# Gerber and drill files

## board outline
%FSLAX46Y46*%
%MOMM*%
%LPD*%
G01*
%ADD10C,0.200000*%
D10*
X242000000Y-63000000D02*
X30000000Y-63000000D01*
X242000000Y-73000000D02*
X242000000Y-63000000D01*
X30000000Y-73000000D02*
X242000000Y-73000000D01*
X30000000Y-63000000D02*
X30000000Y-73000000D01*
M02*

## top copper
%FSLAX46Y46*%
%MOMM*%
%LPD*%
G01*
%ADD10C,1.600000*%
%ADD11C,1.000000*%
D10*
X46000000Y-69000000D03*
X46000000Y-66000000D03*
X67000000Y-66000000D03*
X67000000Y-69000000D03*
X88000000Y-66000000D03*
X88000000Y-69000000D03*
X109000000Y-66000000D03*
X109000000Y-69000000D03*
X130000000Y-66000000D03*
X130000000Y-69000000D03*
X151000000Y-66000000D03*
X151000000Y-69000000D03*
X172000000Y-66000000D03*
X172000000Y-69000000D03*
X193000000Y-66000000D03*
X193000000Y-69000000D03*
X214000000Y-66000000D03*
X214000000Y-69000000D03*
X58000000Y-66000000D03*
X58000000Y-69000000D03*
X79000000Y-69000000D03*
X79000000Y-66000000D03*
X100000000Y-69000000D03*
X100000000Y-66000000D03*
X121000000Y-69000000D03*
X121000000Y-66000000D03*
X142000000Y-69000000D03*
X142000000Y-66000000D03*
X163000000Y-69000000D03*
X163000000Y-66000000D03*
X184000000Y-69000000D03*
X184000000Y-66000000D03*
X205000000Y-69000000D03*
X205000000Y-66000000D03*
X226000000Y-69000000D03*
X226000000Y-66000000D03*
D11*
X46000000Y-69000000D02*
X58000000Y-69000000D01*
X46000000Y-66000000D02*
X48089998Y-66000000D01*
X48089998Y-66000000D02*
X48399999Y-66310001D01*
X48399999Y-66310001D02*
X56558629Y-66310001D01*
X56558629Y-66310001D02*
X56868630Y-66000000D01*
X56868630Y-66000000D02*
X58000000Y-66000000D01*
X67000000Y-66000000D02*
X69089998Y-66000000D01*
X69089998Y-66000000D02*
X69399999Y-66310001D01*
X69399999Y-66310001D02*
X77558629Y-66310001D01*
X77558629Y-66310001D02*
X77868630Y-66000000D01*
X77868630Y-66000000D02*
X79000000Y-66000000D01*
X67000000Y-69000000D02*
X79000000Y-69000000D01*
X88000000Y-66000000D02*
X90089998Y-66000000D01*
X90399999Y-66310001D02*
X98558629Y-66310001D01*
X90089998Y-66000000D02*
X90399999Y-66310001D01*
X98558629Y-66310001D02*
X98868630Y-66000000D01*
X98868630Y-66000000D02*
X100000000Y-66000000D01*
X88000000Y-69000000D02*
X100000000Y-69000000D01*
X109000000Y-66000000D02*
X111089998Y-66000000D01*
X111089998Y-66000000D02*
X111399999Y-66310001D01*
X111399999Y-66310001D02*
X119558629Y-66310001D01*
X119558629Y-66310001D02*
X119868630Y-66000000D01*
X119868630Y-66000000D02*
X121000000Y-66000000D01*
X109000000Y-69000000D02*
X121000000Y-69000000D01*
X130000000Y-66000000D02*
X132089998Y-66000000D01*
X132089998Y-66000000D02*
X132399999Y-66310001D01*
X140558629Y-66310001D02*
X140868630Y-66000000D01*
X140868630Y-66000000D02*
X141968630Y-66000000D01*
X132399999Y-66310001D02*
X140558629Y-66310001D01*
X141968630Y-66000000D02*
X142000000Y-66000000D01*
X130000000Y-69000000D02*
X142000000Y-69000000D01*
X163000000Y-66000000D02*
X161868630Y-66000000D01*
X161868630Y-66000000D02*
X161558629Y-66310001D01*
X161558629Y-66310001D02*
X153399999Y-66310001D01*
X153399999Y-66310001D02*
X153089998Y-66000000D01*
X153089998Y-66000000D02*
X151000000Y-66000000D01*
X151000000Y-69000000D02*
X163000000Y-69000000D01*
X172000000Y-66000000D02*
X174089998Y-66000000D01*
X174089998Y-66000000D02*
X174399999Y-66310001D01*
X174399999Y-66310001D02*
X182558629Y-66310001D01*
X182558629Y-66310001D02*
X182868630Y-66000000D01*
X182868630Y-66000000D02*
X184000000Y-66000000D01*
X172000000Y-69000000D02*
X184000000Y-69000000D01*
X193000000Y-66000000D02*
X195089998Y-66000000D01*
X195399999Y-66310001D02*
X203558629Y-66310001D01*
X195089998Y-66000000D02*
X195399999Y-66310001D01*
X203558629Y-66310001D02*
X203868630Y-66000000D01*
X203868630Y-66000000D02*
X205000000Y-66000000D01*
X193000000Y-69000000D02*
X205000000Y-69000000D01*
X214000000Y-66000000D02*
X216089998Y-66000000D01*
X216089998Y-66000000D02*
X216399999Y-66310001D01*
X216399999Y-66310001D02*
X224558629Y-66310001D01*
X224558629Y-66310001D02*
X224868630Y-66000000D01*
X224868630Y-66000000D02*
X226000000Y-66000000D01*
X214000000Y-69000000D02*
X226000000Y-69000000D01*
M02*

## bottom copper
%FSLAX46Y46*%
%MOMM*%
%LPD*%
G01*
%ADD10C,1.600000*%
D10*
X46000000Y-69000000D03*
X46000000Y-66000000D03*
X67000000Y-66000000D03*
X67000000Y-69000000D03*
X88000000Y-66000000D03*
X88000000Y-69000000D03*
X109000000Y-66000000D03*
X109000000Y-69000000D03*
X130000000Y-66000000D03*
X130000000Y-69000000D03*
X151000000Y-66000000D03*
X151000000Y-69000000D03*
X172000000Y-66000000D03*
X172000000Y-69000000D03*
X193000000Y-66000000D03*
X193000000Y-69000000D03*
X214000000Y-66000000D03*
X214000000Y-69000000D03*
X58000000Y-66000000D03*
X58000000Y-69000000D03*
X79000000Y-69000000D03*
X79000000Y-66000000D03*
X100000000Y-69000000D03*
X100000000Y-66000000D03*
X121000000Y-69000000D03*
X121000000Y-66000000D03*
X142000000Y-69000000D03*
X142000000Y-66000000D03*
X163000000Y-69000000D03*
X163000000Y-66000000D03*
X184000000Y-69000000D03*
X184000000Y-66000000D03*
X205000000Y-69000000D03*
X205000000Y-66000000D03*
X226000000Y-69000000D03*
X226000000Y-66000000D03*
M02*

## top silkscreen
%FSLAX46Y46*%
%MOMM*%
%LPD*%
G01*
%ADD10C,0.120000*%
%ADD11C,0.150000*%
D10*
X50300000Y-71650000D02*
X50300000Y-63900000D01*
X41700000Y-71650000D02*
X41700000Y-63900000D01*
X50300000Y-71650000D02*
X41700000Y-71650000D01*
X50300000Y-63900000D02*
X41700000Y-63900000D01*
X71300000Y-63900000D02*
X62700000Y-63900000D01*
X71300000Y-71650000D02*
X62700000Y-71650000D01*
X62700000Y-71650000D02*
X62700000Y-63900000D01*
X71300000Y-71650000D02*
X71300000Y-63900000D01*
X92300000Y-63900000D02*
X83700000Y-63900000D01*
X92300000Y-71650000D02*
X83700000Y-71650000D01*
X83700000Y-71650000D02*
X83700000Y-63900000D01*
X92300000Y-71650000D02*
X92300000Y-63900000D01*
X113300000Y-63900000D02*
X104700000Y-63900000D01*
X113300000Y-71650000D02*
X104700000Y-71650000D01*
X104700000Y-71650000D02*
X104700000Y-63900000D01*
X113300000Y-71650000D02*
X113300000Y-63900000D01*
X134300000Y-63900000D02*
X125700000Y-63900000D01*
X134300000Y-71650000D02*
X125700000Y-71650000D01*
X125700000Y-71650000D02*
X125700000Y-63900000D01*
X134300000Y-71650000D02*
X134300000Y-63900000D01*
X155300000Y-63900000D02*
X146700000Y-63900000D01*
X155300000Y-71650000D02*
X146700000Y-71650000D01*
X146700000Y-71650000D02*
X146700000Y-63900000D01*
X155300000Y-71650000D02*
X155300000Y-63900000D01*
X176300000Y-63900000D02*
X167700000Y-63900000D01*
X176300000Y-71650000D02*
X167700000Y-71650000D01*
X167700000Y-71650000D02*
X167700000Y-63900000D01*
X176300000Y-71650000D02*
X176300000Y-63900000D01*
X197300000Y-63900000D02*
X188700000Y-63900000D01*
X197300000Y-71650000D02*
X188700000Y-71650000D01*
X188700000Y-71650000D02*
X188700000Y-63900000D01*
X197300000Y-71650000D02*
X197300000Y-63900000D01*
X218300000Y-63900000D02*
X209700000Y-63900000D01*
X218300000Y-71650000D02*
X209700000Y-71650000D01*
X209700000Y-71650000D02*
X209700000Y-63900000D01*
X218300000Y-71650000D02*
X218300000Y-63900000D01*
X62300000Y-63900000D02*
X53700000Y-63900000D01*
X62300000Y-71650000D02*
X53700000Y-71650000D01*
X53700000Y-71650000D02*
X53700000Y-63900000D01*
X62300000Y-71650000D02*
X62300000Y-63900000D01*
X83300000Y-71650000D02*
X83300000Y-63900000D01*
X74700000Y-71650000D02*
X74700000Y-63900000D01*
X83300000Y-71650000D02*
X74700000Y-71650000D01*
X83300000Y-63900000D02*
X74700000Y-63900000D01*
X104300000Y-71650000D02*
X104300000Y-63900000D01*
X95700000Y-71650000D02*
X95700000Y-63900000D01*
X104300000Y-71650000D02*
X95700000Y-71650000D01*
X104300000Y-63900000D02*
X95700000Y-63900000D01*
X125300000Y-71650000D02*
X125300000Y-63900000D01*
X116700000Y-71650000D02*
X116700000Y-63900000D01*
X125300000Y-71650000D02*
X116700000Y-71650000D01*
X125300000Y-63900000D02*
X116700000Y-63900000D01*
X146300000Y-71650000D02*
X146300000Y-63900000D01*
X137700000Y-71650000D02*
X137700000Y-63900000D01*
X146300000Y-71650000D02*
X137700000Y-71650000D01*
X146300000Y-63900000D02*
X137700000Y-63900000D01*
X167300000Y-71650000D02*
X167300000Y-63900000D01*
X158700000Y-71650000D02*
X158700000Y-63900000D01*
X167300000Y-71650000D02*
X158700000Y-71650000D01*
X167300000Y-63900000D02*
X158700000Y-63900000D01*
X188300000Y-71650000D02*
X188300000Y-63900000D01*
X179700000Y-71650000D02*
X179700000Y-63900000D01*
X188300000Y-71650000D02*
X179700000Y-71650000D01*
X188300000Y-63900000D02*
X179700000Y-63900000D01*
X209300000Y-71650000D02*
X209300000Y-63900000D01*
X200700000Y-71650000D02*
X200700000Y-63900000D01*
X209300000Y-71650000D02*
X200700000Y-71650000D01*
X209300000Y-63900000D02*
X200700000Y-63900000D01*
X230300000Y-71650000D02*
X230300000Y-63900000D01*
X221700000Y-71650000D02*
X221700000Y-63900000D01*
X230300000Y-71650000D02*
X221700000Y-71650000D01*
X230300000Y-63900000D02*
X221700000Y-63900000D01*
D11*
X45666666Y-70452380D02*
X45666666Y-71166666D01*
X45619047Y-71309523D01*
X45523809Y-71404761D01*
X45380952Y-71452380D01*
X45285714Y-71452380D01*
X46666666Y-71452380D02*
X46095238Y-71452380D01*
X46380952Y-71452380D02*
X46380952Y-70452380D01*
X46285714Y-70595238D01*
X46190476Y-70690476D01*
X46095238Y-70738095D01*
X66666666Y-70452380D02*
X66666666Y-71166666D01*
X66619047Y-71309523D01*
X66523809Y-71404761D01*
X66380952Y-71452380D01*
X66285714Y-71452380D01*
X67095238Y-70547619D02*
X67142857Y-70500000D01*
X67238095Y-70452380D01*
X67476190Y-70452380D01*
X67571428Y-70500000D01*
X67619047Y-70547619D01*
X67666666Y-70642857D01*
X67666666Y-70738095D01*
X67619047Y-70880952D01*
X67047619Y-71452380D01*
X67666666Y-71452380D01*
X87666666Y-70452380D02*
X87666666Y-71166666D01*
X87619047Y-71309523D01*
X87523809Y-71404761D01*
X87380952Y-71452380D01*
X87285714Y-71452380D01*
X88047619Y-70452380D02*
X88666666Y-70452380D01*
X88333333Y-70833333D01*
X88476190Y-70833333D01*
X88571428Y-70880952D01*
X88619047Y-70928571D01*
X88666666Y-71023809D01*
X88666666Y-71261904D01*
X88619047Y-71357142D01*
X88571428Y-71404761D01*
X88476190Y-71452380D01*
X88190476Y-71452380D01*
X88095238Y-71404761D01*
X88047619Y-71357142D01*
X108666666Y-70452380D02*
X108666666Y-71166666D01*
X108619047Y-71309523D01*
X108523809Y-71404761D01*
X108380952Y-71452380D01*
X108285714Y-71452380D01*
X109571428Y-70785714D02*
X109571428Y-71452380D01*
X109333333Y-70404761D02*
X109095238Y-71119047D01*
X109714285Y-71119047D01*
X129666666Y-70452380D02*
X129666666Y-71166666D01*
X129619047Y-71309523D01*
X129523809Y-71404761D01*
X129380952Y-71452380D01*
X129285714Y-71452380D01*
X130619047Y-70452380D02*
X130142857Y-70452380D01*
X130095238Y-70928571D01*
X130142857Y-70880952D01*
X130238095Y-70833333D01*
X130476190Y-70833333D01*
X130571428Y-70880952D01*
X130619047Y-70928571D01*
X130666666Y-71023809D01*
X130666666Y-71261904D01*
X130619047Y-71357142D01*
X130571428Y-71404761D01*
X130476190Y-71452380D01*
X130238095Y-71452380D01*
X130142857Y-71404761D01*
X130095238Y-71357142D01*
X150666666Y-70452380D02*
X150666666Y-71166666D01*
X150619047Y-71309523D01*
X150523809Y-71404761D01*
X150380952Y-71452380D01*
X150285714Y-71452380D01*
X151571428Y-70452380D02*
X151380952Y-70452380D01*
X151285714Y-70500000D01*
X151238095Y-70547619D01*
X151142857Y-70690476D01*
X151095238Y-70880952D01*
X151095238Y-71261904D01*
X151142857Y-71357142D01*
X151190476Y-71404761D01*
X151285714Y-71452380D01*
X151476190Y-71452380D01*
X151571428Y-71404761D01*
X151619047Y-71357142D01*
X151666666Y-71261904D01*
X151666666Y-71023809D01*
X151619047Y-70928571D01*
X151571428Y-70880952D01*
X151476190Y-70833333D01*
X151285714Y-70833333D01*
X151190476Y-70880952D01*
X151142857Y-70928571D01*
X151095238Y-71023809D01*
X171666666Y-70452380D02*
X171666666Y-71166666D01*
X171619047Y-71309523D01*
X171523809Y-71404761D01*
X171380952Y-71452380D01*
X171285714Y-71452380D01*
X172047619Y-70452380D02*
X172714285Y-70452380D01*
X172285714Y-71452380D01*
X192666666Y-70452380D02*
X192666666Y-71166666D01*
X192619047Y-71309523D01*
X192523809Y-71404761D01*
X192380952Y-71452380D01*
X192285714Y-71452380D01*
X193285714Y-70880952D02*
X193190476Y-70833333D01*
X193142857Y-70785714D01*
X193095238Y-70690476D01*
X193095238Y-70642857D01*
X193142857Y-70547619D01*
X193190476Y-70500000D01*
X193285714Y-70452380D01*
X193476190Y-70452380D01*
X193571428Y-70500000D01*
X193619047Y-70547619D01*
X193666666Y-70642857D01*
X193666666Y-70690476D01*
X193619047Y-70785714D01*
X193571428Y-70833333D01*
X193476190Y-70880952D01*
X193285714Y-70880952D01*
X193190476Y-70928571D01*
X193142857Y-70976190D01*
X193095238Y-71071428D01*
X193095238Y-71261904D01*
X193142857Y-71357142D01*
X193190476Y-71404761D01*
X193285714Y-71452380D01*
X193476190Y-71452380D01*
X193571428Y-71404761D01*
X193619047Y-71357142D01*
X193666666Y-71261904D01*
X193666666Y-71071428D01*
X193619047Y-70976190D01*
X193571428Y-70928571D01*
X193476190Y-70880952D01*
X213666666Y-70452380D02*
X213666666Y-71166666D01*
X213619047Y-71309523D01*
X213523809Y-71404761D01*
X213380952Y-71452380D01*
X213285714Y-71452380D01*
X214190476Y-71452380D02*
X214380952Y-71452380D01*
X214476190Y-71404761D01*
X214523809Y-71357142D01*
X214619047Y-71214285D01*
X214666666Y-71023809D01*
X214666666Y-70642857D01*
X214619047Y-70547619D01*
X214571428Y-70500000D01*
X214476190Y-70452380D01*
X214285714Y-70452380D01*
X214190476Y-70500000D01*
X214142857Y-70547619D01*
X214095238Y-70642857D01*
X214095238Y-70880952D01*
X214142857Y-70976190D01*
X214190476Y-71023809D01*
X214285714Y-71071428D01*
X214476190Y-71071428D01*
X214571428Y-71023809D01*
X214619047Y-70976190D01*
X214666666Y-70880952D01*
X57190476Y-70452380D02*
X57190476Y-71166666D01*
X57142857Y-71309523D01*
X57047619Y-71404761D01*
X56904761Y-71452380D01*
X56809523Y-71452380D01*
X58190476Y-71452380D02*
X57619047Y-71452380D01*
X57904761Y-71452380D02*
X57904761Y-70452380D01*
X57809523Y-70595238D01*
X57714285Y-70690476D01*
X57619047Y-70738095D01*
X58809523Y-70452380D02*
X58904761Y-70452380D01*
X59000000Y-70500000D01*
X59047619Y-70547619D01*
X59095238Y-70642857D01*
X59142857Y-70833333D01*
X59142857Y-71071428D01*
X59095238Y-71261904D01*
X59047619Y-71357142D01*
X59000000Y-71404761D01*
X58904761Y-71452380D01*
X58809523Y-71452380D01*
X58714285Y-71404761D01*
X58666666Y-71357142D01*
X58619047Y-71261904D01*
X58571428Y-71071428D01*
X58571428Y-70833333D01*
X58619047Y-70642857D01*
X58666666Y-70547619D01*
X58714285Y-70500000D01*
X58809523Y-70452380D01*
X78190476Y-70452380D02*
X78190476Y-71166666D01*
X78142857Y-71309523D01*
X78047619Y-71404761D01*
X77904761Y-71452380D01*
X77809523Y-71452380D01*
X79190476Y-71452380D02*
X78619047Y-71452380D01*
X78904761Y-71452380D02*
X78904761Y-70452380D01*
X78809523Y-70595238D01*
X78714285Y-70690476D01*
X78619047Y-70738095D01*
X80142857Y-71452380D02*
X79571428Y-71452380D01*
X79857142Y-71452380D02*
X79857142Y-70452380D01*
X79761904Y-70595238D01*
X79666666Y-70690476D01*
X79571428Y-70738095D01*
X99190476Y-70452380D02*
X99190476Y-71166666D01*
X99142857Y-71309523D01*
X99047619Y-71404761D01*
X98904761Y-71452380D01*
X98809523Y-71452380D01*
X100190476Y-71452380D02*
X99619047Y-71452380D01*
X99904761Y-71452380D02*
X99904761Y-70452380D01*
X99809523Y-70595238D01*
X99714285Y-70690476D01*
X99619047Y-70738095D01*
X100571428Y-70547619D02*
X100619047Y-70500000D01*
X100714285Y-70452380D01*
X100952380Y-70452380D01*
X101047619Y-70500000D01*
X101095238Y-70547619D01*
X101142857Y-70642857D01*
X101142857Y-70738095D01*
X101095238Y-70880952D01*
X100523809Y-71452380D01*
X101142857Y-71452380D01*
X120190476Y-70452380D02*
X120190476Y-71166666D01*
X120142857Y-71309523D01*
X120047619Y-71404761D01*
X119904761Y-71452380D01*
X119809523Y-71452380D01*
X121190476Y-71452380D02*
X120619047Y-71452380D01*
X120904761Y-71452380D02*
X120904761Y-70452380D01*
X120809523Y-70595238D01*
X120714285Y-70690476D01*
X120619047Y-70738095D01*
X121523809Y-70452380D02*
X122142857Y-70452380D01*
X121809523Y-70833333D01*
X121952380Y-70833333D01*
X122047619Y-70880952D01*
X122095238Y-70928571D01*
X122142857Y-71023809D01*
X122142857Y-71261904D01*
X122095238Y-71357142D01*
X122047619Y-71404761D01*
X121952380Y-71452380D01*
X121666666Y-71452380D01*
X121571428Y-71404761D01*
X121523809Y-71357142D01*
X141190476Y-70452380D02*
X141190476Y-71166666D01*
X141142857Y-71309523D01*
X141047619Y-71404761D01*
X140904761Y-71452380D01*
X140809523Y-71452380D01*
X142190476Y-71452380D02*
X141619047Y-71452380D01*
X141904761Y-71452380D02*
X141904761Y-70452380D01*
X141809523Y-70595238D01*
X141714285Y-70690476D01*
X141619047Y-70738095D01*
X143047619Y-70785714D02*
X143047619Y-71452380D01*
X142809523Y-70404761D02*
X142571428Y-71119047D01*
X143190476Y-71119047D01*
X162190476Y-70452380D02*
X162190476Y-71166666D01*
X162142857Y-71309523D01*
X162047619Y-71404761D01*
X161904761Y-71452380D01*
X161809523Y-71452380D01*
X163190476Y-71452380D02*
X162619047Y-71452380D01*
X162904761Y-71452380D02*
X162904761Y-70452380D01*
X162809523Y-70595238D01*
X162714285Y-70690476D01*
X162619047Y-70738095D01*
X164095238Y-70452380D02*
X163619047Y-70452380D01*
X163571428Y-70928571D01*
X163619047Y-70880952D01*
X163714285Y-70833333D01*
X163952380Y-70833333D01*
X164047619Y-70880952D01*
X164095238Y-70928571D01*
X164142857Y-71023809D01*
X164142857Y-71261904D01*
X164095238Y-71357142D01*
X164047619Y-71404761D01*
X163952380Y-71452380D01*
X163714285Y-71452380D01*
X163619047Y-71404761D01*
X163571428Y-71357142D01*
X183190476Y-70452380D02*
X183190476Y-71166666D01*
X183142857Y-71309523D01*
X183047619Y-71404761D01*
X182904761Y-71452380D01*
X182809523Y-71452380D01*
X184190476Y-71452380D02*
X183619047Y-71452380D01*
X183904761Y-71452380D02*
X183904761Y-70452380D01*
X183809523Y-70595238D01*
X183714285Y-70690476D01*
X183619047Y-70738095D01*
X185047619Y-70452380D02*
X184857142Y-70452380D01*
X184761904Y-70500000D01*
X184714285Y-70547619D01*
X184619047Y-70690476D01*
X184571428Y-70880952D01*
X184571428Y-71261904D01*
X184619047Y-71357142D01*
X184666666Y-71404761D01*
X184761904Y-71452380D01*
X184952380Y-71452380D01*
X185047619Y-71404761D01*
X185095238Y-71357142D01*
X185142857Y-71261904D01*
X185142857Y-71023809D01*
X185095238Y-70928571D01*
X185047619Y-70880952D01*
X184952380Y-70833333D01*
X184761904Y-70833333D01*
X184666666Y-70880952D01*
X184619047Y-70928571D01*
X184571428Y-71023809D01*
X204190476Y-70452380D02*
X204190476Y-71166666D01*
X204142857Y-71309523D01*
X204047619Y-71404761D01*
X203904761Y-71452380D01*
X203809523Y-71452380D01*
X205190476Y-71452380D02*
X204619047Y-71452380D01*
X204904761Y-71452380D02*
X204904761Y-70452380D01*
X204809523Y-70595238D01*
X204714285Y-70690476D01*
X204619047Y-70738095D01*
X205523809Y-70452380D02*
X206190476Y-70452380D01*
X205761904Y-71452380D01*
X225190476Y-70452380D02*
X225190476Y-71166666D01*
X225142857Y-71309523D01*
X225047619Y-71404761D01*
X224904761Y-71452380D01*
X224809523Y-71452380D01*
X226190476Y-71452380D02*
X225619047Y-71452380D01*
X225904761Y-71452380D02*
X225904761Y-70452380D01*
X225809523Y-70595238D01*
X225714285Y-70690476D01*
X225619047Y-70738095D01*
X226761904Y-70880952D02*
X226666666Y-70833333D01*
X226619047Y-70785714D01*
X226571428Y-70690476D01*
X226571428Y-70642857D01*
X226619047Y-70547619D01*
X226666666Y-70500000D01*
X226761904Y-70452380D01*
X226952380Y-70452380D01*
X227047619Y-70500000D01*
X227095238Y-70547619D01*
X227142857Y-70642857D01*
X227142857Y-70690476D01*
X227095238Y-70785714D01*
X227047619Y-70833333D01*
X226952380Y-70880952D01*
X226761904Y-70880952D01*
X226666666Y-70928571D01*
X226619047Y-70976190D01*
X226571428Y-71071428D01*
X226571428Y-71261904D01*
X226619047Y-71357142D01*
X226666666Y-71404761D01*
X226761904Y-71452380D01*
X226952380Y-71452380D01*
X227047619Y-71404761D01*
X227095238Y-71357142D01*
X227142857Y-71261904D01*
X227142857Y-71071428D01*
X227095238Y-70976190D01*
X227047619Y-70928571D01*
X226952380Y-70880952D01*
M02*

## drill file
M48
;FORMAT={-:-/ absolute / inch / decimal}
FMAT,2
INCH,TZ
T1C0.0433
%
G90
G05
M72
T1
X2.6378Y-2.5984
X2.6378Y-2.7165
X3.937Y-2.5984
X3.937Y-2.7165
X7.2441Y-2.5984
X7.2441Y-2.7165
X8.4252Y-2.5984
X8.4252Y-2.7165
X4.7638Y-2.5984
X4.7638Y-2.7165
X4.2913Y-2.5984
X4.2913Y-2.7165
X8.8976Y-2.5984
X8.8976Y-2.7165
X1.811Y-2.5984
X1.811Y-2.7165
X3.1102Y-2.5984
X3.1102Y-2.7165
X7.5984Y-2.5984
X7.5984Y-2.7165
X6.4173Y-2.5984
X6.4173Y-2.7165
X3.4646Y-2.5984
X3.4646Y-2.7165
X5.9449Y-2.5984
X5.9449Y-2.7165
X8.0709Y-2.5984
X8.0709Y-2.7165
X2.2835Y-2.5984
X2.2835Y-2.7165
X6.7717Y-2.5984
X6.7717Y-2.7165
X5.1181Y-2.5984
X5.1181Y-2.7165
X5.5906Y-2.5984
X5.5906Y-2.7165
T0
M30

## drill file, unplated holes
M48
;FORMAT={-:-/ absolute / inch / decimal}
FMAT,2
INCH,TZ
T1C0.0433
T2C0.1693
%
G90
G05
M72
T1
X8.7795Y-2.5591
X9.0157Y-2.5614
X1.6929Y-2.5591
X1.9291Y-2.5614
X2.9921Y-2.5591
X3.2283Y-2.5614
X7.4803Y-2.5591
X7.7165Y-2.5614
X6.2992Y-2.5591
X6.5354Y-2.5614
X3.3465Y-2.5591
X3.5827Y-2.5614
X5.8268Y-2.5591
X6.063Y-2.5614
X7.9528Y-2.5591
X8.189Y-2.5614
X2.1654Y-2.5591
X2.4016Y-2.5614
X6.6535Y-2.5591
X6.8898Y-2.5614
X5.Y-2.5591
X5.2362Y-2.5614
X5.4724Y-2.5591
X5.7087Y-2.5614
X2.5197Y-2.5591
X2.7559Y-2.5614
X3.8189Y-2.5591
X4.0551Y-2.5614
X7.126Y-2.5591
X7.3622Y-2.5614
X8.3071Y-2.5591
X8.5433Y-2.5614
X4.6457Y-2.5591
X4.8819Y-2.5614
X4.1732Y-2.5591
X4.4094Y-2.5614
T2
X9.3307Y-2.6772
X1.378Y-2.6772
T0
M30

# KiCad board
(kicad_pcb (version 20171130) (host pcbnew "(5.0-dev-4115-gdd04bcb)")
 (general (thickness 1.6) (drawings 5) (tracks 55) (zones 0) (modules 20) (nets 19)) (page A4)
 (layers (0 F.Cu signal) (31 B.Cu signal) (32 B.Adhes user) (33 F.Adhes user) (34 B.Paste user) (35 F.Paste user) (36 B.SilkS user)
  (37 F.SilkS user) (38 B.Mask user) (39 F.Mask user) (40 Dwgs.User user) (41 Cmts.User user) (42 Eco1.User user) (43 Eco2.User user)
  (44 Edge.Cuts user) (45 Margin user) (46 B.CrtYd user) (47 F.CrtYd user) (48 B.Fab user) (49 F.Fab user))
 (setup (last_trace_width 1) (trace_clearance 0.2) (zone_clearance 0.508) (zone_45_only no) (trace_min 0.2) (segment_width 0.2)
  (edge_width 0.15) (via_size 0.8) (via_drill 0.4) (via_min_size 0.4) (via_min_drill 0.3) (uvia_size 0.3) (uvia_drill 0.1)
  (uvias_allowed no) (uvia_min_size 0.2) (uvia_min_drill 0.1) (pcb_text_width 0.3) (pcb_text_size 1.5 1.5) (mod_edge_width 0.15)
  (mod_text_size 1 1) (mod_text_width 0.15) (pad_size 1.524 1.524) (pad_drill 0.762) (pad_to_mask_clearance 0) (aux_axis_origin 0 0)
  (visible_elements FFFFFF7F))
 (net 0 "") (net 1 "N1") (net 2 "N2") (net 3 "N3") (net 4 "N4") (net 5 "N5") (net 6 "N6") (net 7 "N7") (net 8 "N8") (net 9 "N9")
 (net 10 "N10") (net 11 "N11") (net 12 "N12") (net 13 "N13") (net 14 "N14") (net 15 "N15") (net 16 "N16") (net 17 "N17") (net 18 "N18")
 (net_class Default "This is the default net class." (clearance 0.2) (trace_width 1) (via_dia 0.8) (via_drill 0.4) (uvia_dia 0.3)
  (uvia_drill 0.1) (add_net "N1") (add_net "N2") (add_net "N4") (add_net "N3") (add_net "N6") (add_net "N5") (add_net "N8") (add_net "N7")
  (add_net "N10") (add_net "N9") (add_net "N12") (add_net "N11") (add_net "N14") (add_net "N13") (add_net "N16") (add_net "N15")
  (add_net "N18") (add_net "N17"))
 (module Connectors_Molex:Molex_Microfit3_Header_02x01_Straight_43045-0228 (layer F.Cu) (at 46 69)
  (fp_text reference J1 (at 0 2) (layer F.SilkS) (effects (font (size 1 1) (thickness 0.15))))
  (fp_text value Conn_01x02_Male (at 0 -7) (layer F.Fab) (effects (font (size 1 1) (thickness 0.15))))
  (fp_line (start 4.3 2.65) (end 4.3 -5.1) (layer F.SilkS) (width 0.12))
  (fp_line (start -4.3 2.65) (end -4.3 -5.1) (layer F.SilkS) (width 0.12))
  (fp_line (start 4.3 2.65) (end -4.3 2.65) (layer F.SilkS) (width 0.12))
  (fp_line (start 4.3 -5.1) (end -4.3 -5.1) (layer F.SilkS) (width 0.12))
  (pad "" np_thru_hole circle (at -3 -4) (size 1.1 1.1) (drill 1.1) (layers *.Cu *.Mask))
  (pad 1 thru_hole circle (at 0 0) (size 1.6 1.6) (drill 1.1) (layers *.Cu *.Mask) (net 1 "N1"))
  (pad 2 thru_hole circle (at 0 -3) (size 1.6 1.6) (drill 1.1) (layers *.Cu *.Mask) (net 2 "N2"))
  (pad "" np_thru_hole circle (at 3 -3.94) (size 1.1 1.1) (drill 1.1) (layers *.Cu *.Mask)))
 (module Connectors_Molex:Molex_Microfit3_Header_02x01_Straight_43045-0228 (layer F.Cu) (at 67 69)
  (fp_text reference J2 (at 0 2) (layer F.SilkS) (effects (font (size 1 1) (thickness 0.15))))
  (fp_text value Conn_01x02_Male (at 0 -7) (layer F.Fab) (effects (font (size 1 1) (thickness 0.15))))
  (fp_line (start 4.3 -5.1) (end -4.3 -5.1) (layer F.SilkS) (width 0.12))
  (fp_line (start 4.3 2.65) (end -4.3 2.65) (layer F.SilkS) (width 0.12))
  (fp_line (start -4.3 2.65) (end -4.3 -5.1) (layer F.SilkS) (width 0.12))
  (fp_line (start 4.3 2.65) (end 4.3 -5.1) (layer F.SilkS) (width 0.12))
  (pad "" np_thru_hole circle (at 3 -3.94) (size 1.1 1.1) (drill 1.1) (layers *.Cu *.Mask))
  (pad 2 thru_hole circle (at 0 -3) (size 1.6 1.6) (drill 1.1) (layers *.Cu *.Mask) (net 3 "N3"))
  (pad 1 thru_hole circle (at 0 0) (size 1.6 1.6) (drill 1.1) (layers *.Cu *.Mask) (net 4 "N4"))
  (pad "" np_thru_hole circle (at -3 -4) (size 1.1 1.1) (drill 1.1) (layers *.Cu *.Mask)))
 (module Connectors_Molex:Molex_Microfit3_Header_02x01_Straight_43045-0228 (layer F.Cu) (at 88 69)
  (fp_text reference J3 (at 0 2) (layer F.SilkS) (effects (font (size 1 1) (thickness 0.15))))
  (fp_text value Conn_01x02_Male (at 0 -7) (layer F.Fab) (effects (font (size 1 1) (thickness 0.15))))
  (fp_line (start 4.3 -5.1) (end -4.3 -5.1) (layer F.SilkS) (width 0.12))
  (fp_line (start 4.3 2.65) (end -4.3 2.65) (layer F.SilkS) (width 0.12))
  (fp_line (start -4.3 2.65) (end -4.3 -5.1) (layer F.SilkS) (width 0.12))
  (fp_line (start 4.3 2.65) (end 4.3 -5.1) (layer F.SilkS) (width 0.12))
  (pad "" np_thru_hole circle (at 3 -3.94) (size 1.1 1.1) (drill 1.1) (layers *.Cu *.Mask))
  (pad 2 thru_hole circle (at 0 -3) (size 1.6 1.6) (drill 1.1) (layers *.Cu *.Mask) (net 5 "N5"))
  (pad 1 thru_hole circle (at 0 0) (size 1.6 1.6) (drill 1.1) (layers *.Cu *.Mask) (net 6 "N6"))
  (pad "" np_thru_hole circle (at -3 -4) (size 1.1 1.1) (drill 1.1) (layers *.Cu *.Mask)))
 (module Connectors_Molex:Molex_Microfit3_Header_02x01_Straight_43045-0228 (layer F.Cu) (at 109 69)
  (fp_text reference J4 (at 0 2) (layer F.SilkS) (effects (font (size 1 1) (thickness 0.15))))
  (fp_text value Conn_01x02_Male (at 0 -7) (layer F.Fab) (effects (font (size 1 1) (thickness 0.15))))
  (fp_line (start 4.3 -5.1) (end -4.3 -5.1) (layer F.SilkS) (width 0.12))
  (fp_line (start 4.3 2.65) (end -4.3 2.65) (layer F.SilkS) (width 0.12))
  (fp_line (start -4.3 2.65) (end -4.3 -5.1) (layer F.SilkS) (width 0.12))
  (fp_line (start 4.3 2.65) (end 4.3 -5.1) (layer F.SilkS) (width 0.12))
  (pad "" np_thru_hole circle (at 3 -3.94) (size 1.1 1.1) (drill 1.1) (layers *.Cu *.Mask))
  (pad 2 thru_hole circle (at 0 -3) (size 1.6 1.6) (drill 1.1) (layers *.Cu *.Mask) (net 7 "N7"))
  (pad 1 thru_hole circle (at 0 0) (size 1.6 1.6) (drill 1.1) (layers *.Cu *.Mask) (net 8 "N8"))
  (pad "" np_thru_hole circle (at -3 -4) (size 1.1 1.1) (drill 1.1) (layers *.Cu *.Mask)))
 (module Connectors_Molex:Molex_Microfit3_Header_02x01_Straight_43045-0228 (layer F.Cu) (at 130 69)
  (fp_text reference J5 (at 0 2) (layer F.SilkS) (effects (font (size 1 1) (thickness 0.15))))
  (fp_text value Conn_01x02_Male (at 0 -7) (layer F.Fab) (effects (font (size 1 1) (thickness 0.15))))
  (fp_line (start 4.3 -5.1) (end -4.3 -5.1) (layer F.SilkS) (width 0.12))
  (fp_line (start 4.3 2.65) (end -4.3 2.65) (layer F.SilkS) (width 0.12))
  (fp_line (start -4.3 2.65) (end -4.3 -5.1) (layer F.SilkS) (width 0.12))
  (fp_line (start 4.3 2.65) (end 4.3 -5.1) (layer F.SilkS) (width 0.12))
  (pad "" np_thru_hole circle (at 3 -3.94) (size 1.1 1.1) (drill 1.1) (layers *.Cu *.Mask))
  (pad 2 thru_hole circle (at 0 -3) (size 1.6 1.6) (drill 1.1) (layers *.Cu *.Mask) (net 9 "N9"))
  (pad 1 thru_hole circle (at 0 0) (size 1.6 1.6) (drill 1.1) (layers *.Cu *.Mask) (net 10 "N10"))
  (pad "" np_thru_hole circle (at -3 -4) (size 1.1 1.1) (drill 1.1) (layers *.Cu *.Mask)))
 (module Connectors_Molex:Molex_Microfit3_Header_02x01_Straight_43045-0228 (layer F.Cu) (at 151 69)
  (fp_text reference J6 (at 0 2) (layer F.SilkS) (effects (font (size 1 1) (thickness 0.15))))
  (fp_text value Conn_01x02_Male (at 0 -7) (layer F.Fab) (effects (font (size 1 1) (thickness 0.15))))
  (fp_line (start 4.3 -5.1) (end -4.3 -5.1) (layer F.SilkS) (width 0.12))
  (fp_line (start 4.3 2.65) (end -4.3 2.65) (layer F.SilkS) (width 0.12))
  (fp_line (start -4.3 2.65) (end -4.3 -5.1) (layer F.SilkS) (width 0.12))
  (fp_line (start 4.3 2.65) (end 4.3 -5.1) (layer F.SilkS) (width 0.12))
  (pad "" np_thru_hole circle (at 3 -3.94) (size 1.1 1.1) (drill 1.1) (layers *.Cu *.Mask))
  (pad 2 thru_hole circle (at 0 -3) (size 1.6 1.6) (drill 1.1) (layers *.Cu *.Mask) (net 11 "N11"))
  (pad 1 thru_hole circle (at 0 0) (size 1.6 1.6) (drill 1.1) (layers *.Cu *.Mask) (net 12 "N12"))
  (pad "" np_thru_hole circle (at -3 -4) (size 1.1 1.1) (drill 1.1) (layers *.Cu *.Mask)))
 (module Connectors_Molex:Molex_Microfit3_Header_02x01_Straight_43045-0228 (layer F.Cu) (at 172 69)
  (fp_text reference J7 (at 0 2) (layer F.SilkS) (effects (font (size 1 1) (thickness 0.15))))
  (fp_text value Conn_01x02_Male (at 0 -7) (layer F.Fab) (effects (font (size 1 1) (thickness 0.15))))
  (fp_line (start 4.3 -5.1) (end -4.3 -5.1) (layer F.SilkS) (width 0.12))
  (fp_line (start 4.3 2.65) (end -4.3 2.65) (layer F.SilkS) (width 0.12))
  (fp_line (start -4.3 2.65) (end -4.3 -5.1) (layer F.SilkS) (width 0.12))
  (fp_line (start 4.3 2.65) (end 4.3 -5.1) (layer F.SilkS) (width 0.12))
  (pad "" np_thru_hole circle (at 3 -3.94) (size 1.1 1.1) (drill 1.1) (layers *.Cu *.Mask))
  (pad 2 thru_hole circle (at 0 -3) (size 1.6 1.6) (drill 1.1) (layers *.Cu *.Mask) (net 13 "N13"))
  (pad 1 thru_hole circle (at 0 0) (size 1.6 1.6) (drill 1.1) (layers *.Cu *.Mask) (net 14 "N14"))
  (pad "" np_thru_hole circle (at -3 -4) (size 1.1 1.1) (drill 1.1) (layers *.Cu *.Mask)))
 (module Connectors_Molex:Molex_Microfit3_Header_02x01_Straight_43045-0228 (layer F.Cu) (at 193 69)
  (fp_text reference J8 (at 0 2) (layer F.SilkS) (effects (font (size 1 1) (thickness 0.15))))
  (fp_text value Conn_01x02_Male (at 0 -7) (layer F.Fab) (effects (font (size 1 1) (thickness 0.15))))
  (fp_line (start 4.3 -5.1) (end -4.3 -5.1) (layer F.SilkS) (width 0.12))
  (fp_line (start 4.3 2.65) (end -4.3 2.65) (layer F.SilkS) (width 0.12))
  (fp_line (start -4.3 2.65) (end -4.3 -5.1) (layer F.SilkS) (width 0.12))
  (fp_line (start 4.3 2.65) (end 4.3 -5.1) (layer F.SilkS) (width 0.12))
  (pad "" np_thru_hole circle (at 3 -3.94) (size 1.1 1.1) (drill 1.1) (layers *.Cu *.Mask))
  (pad 2 thru_hole circle (at 0 -3) (size 1.6 1.6) (drill 1.1) (layers *.Cu *.Mask) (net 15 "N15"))
  (pad 1 thru_hole circle (at 0 0) (size 1.6 1.6) (drill 1.1) (layers *.Cu *.Mask) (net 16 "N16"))
  (pad "" np_thru_hole circle (at -3 -4) (size 1.1 1.1) (drill 1.1) (layers *.Cu *.Mask)))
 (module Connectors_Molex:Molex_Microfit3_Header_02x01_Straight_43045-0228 (layer F.Cu) (at 214 69)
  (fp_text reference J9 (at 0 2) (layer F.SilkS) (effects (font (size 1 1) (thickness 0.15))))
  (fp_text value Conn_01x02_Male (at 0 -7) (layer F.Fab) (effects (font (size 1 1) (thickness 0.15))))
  (fp_line (start 4.3 -5.1) (end -4.3 -5.1) (layer F.SilkS) (width 0.12))
  (fp_line (start 4.3 2.65) (end -4.3 2.65) (layer F.SilkS) (width 0.12))
  (fp_line (start -4.3 2.65) (end -4.3 -5.1) (layer F.SilkS) (width 0.12))
  (fp_line (start 4.3 2.65) (end 4.3 -5.1) (layer F.SilkS) (width 0.12))
  (pad "" np_thru_hole circle (at 3 -3.94) (size 1.1 1.1) (drill 1.1) (layers *.Cu *.Mask))
  (pad 2 thru_hole circle (at 0 -3) (size 1.6 1.6) (drill 1.1) (layers *.Cu *.Mask) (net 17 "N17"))
  (pad 1 thru_hole circle (at 0 0) (size 1.6 1.6) (drill 1.1) (layers *.Cu *.Mask) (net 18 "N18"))
  (pad "" np_thru_hole circle (at -3 -4) (size 1.1 1.1) (drill 1.1) (layers *.Cu *.Mask)))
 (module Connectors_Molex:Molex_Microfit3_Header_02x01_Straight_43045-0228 (layer F.Cu) (at 58 69)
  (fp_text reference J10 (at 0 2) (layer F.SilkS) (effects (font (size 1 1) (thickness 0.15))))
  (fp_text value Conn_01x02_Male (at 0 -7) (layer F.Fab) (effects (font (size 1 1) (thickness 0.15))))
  (fp_line (start 4.3 -5.1) (end -4.3 -5.1) (layer F.SilkS) (width 0.12))
  (fp_line (start 4.3 2.65) (end -4.3 2.65) (layer F.SilkS) (width 0.12))
  (fp_line (start -4.3 2.65) (end -4.3 -5.1) (layer F.SilkS) (width 0.12))
  (fp_line (start 4.3 2.65) (end 4.3 -5.1) (layer F.SilkS) (width 0.12))
  (pad "" np_thru_hole circle (at 3 -3.94) (size 1.1 1.1) (drill 1.1) (layers *.Cu *.Mask))
  (pad 2 thru_hole circle (at 0 -3) (size 1.6 1.6) (drill 1.1) (layers *.Cu *.Mask) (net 2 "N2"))
  (pad 1 thru_hole circle (at 0 0) (size 1.6 1.6) (drill 1.1) (layers *.Cu *.Mask) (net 1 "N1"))
  (pad "" np_thru_hole circle (at -3 -4) (size 1.1 1.1) (drill 1.1) (layers *.Cu *.Mask)))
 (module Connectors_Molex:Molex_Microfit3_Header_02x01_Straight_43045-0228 (layer F.Cu) (at 79 69)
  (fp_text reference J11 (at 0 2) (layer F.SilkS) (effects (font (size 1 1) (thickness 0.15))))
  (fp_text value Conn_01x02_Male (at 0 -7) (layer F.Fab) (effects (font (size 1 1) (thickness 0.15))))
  (fp_line (start 4.3 2.65) (end 4.3 -5.1) (layer F.SilkS) (width 0.12))
  (fp_line (start -4.3 2.65) (end -4.3 -5.1) (layer F.SilkS) (width 0.12))
  (fp_line (start 4.3 2.65) (end -4.3 2.65) (layer F.SilkS) (width 0.12))
  (fp_line (start 4.3 -5.1) (end -4.3 -5.1) (layer F.SilkS) (width 0.12))
  (pad "" np_thru_hole circle (at -3 -4) (size 1.1 1.1) (drill 1.1) (layers *.Cu *.Mask))
  (pad 1 thru_hole circle (at 0 0) (size 1.6 1.6) (drill 1.1) (layers *.Cu *.Mask) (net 4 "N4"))
  (pad 2 thru_hole circle (at 0 -3) (size 1.6 1.6) (drill 1.1) (layers *.Cu *.Mask) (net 3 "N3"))
  (pad "" np_thru_hole circle (at 3 -3.94) (size 1.1 1.1) (drill 1.1) (layers *.Cu *.Mask)))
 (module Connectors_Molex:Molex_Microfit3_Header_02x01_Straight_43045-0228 (layer F.Cu) (at 100 69)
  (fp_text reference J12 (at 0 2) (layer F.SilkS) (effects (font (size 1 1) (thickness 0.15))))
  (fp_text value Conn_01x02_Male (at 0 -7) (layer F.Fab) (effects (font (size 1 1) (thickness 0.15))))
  (fp_line (start 4.3 2.65) (end 4.3 -5.1) (layer F.SilkS) (width 0.12))
  (fp_line (start -4.3 2.65) (end -4.3 -5.1) (layer F.SilkS) (width 0.12))
  (fp_line (start 4.3 2.65) (end -4.3 2.65) (layer F.SilkS) (width 0.12))
  (fp_line (start 4.3 -5.1) (end -4.3 -5.1) (layer F.SilkS) (width 0.12))
  (pad "" np_thru_hole circle (at -3 -4) (size 1.1 1.1) (drill 1.1) (layers *.Cu *.Mask))
  (pad 1 thru_hole circle (at 0 0) (size 1.6 1.6) (drill 1.1) (layers *.Cu *.Mask) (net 6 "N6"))
  (pad 2 thru_hole circle (at 0 -3) (size 1.6 1.6) (drill 1.1) (layers *.Cu *.Mask) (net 5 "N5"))
  (pad "" np_thru_hole circle (at 3 -3.94) (size 1.1 1.1) (drill 1.1) (layers *.Cu *.Mask)))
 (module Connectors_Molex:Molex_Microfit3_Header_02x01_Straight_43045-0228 (layer F.Cu) (at 121 69)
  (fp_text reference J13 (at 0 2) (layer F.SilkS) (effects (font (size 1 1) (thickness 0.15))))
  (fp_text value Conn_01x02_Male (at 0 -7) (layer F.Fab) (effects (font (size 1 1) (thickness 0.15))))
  (fp_line (start 4.3 2.65) (end 4.3 -5.1) (layer F.SilkS) (width 0.12))
  (fp_line (start -4.3 2.65) (end -4.3 -5.1) (layer F.SilkS) (width 0.12))
  (fp_line (start 4.3 2.65) (end -4.3 2.65) (layer F.SilkS) (width 0.12))
  (fp_line (start 4.3 -5.1) (end -4.3 -5.1) (layer F.SilkS) (width 0.12))
  (pad "" np_thru_hole circle (at -3 -4) (size 1.1 1.1) (drill 1.1) (layers *.Cu *.Mask))
  (pad 1 thru_hole circle (at 0 0) (size 1.6 1.6) (drill 1.1) (layers *.Cu *.Mask) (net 8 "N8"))
  (pad 2 thru_hole circle (at 0 -3) (size 1.6 1.6) (drill 1.1) (layers *.Cu *.Mask) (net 7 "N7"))
  (pad "" np_thru_hole circle (at 3 -3.94) (size 1.1 1.1) (drill 1.1) (layers *.Cu *.Mask)))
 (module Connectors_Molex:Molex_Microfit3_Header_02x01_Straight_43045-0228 (layer F.Cu) (at 142 69)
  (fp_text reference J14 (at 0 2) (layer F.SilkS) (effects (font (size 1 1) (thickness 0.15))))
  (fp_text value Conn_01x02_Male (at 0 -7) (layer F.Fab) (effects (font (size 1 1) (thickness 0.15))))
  (fp_line (start 4.3 2.65) (end 4.3 -5.1) (layer F.SilkS) (width 0.12))
  (fp_line (start -4.3 2.65) (end -4.3 -5.1) (layer F.SilkS) (width 0.12))
  (fp_line (start 4.3 2.65) (end -4.3 2.65) (layer F.SilkS) (width 0.12))
  (fp_line (start 4.3 -5.1) (end -4.3 -5.1) (layer F.SilkS) (width 0.12))
  (pad "" np_thru_hole circle (at -3 -4) (size 1.1 1.1) (drill 1.1) (layers *.Cu *.Mask))
  (pad 1 thru_hole circle (at 0 0) (size 1.6 1.6) (drill 1.1) (layers *.Cu *.Mask) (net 10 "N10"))
  (pad 2 thru_hole circle (at 0 -3) (size 1.6 1.6) (drill 1.1) (layers *.Cu *.Mask) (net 9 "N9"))
  (pad "" np_thru_hole circle (at 3 -3.94) (size 1.1 1.1) (drill 1.1) (layers *.Cu *.Mask)))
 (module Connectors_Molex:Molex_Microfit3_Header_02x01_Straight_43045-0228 (layer F.Cu) (at 163 69)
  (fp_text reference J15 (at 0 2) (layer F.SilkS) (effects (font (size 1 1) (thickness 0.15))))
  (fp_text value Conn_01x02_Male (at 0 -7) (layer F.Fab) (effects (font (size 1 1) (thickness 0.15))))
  (fp_line (start 4.3 2.65) (end 4.3 -5.1) (layer F.SilkS) (width 0.12))
  (fp_line (start -4.3 2.65) (end -4.3 -5.1) (layer F.SilkS) (width 0.12))
  (fp_line (start 4.3 2.65) (end -4.3 2.65) (layer F.SilkS) (width 0.12))
  (fp_line (start 4.3 -5.1) (end -4.3 -5.1) (layer F.SilkS) (width 0.12))
  (pad "" np_thru_hole circle (at -3 -4) (size 1.1 1.1) (drill 1.1) (layers *.Cu *.Mask))
  (pad 1 thru_hole circle (at 0 0) (size 1.6 1.6) (drill 1.1) (layers *.Cu *.Mask) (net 12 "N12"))
  (pad 2 thru_hole circle (at 0 -3) (size 1.6 1.6) (drill 1.1) (layers *.Cu *.Mask) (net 11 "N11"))
  (pad "" np_thru_hole circle (at 3 -3.94) (size 1.1 1.1) (drill 1.1) (layers *.Cu *.Mask)))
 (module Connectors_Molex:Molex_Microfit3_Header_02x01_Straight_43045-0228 (layer F.Cu) (at 184 69)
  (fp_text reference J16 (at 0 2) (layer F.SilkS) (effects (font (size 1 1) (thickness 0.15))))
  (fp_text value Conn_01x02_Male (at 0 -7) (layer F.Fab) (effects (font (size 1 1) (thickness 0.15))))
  (fp_line (start 4.3 2.65) (end 4.3 -5.1) (layer F.SilkS) (width 0.12))
  (fp_line (start -4.3 2.65) (end -4.3 -5.1) (layer F.SilkS) (width 0.12))
  (fp_line (start 4.3 2.65) (end -4.3 2.65) (layer F.SilkS) (width 0.12))
  (fp_line (start 4.3 -5.1) (end -4.3 -5.1) (layer F.SilkS) (width 0.12))
  (pad "" np_thru_hole circle (at -3 -4) (size 1.1 1.1) (drill 1.1) (layers *.Cu *.Mask))
  (pad 1 thru_hole circle (at 0 0) (size 1.6 1.6) (drill 1.1) (layers *.Cu *.Mask) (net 14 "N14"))
  (pad 2 thru_hole circle (at 0 -3) (size 1.6 1.6) (drill 1.1) (layers *.Cu *.Mask) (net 13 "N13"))
  (pad "" np_thru_hole circle (at 3 -3.94) (size 1.1 1.1) (drill 1.1) (layers *.Cu *.Mask)))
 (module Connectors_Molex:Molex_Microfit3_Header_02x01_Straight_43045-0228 (layer F.Cu) (at 205 69)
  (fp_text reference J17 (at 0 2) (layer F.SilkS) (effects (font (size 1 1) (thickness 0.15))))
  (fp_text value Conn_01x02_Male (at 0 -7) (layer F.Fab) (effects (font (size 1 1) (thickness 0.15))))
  (fp_line (start 4.3 2.65) (end 4.3 -5.1) (layer F.SilkS) (width 0.12))
  (fp_line (start -4.3 2.65) (end -4.3 -5.1) (layer F.SilkS) (width 0.12))
  (fp_line (start 4.3 2.65) (end -4.3 2.65) (layer F.SilkS) (width 0.12))
  (fp_line (start 4.3 -5.1) (end -4.3 -5.1) (layer F.SilkS) (width 0.12))
  (pad "" np_thru_hole circle (at -3 -4) (size 1.1 1.1) (drill 1.1) (layers *.Cu *.Mask))
  (pad 1 thru_hole circle (at 0 0) (size 1.6 1.6) (drill 1.1) (layers *.Cu *.Mask) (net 16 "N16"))
  (pad 2 thru_hole circle (at 0 -3) (size 1.6 1.6) (drill 1.1) (layers *.Cu *.Mask) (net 15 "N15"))
  (pad "" np_thru_hole circle (at 3 -3.94) (size 1.1 1.1) (drill 1.1) (layers *.Cu *.Mask)))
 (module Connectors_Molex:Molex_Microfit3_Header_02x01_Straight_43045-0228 (layer F.Cu) (at 226 69)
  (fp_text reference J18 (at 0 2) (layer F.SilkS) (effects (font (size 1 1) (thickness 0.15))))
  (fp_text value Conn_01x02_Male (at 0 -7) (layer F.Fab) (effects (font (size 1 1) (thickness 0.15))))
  (fp_line (start 4.3 2.65) (end 4.3 -5.1) (layer F.SilkS) (width 0.12))
  (fp_line (start -4.3 2.65) (end -4.3 -5.1) (layer F.SilkS) (width 0.12))
  (fp_line (start 4.3 2.65) (end -4.3 2.65) (layer F.SilkS) (width 0.12))
  (fp_line (start 4.3 -5.1) (end -4.3 -5.1) (layer F.SilkS) (width 0.12))
  (pad "" np_thru_hole circle (at -3 -4) (size 1.1 1.1) (drill 1.1) (layers *.Cu *.Mask))
  (pad 1 thru_hole circle (at 0 0) (size 1.6 1.6) (drill 1.1) (layers *.Cu *.Mask) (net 18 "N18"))
  (pad 2 thru_hole circle (at 0 -3) (size 1.6 1.6) (drill 1.1) (layers *.Cu *.Mask) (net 17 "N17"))
  (pad "" np_thru_hole circle (at 3 -3.94) (size 1.1 1.1) (drill 1.1) (layers *.Cu *.Mask)))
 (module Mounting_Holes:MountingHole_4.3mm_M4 (layer F.Cu) (at 35 68)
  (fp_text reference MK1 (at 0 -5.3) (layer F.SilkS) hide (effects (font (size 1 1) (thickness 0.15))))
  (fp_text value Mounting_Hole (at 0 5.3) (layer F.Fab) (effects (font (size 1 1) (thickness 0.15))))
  (pad 1 np_thru_hole circle (at 0 0) (size 4.3 4.3) (drill 4.3) (layers *.Cu *.Mask)))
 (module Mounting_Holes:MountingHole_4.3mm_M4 (layer F.Cu) (at 237 68)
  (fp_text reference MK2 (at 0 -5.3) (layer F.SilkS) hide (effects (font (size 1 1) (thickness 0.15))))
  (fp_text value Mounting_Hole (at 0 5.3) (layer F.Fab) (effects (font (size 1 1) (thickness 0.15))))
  (pad 1 np_thru_hole circle (at 0 0) (size 4.3 4.3) (drill 4.3) (layers *.Cu *.Mask)))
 (gr_line (start 242 63) (end 30 63) (layer Edge.Cuts) (width 0.2))
 (gr_line (start 242 73) (end 242 63) (layer Edge.Cuts) (width 0.2))
 (gr_line (start 30 73) (end 242 73) (layer Edge.Cuts) (width 0.2))
 (gr_line (start 30 63) (end 30 73) (layer Edge.Cuts) (width 0.2))
 (segment (start 46 69) (end 58 69) (width 1) (layer F.Cu) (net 1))
 (segment (start 46 66) (end 48.089998 66) (width 1) (layer F.Cu) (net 2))
 (segment (start 48.089998 66) (end 48.399999 66.310001) (width 1) (layer F.Cu) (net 2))
 (segment (start 48.399999 66.310001) (end 56.558629 66.310001) (width 1) (layer F.Cu) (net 2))
 (segment (start 56.558629 66.310001) (end 56.86863 66) (width 1) (layer F.Cu) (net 2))
 (segment (start 56.86863 66) (end 58 66) (width 1) (layer F.Cu) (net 2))
 (segment (start 67 66) (end 69.089998 66) (width 1) (layer F.Cu) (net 3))
 (segment (start 69.089998 66) (end 69.399999 66.310001) (width 1) (layer F.Cu) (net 3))
 (segment (start 69.399999 66.310001) (end 77.558629 66.310001) (width 1) (layer F.Cu) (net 3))
 (segment (start 77.558629 66.310001) (end 77.86863 66) (width 1) (layer F.Cu) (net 3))
 (segment (start 77.86863 66) (end 79 66) (width 1) (layer F.Cu) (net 3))
 (segment (start 67 69) (end 79 69) (width 1) (layer F.Cu) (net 4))
 (segment (start 88 66) (end 90.089998 66) (width 1) (layer F.Cu) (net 5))
 (segment (start 90.399999 66.310001) (end 98.558629 66.310001) (width 1) (layer F.Cu) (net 5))
 (segment (start 90.089998 66) (end 90.399999 66.310001) (width 1) (layer F.Cu) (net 5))
 (segment (start 98.558629 66.310001) (end 98.86863 66) (width 1) (layer F.Cu) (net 5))
 (segment (start 98.86863 66) (end 100 66) (width 1) (layer F.Cu) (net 5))
 (segment (start 88 69) (end 100 69) (width 1) (layer F.Cu) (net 6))
 (segment (start 109 66) (end 111.089998 66) (width 1) (layer F.Cu) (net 7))
 (segment (start 111.089998 66) (end 111.399999 66.310001) (width 1) (layer F.Cu) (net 7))
 (segment (start 111.399999 66.310001) (end 119.558629 66.310001) (width 1) (layer F.Cu) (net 7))
 (segment (start 119.558629 66.310001) (end 119.86863 66) (width 1) (layer F.Cu) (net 7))
 (segment (start 119.86863 66) (end 121 66) (width 1) (layer F.Cu) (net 7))
 (segment (start 109 69) (end 121 69) (width 1) (layer F.Cu) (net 8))
 (segment (start 130 66) (end 132.089998 66) (width 1) (layer F.Cu) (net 9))
 (segment (start 132.089998 66) (end 132.399999 66.310001) (width 1) (layer F.Cu) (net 9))
 (segment (start 140.558629 66.310001) (end 140.86863 66) (width 1) (layer F.Cu) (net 9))
 (segment (start 140.86863 66) (end 141.96863 66) (width 1) (layer F.Cu) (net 9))
 (segment (start 132.399999 66.310001) (end 140.558629 66.310001) (width 1) (layer F.Cu) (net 9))
 (segment (start 141.96863 66) (end 142 66) (width 1) (layer F.Cu) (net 9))
 (segment (start 130 69) (end 142 69) (width 1) (layer F.Cu) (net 10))
 (segment (start 163 66) (end 161.86863 66) (width 1) (layer F.Cu) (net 11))
 (segment (start 161.86863 66) (end 161.558629 66.310001) (width 1) (layer F.Cu) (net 11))
 (segment (start 161.558629 66.310001) (end 153.399999 66.310001) (width 1) (layer F.Cu) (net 11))
 (segment (start 153.399999 66.310001) (end 153.089998 66) (width 1) (layer F.Cu) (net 11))
 (segment (start 153.089998 66) (end 151 66) (width 1) (layer F.Cu) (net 11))
 (segment (start 151 69) (end 163 69) (width 1) (layer F.Cu) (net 12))
 (segment (start 172 66) (end 174.089998 66) (width 1) (layer F.Cu) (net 13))
 (segment (start 174.089998 66) (end 174.399999 66.310001) (width 1) (layer F.Cu) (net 13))
 (segment (start 174.399999 66.310001) (end 182.558629 66.310001) (width 1) (layer F.Cu) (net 13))
 (segment (start 182.558629 66.310001) (end 182.86863 66) (width 1) (layer F.Cu) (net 13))
 (segment (start 182.86863 66) (end 184 66) (width 1) (layer F.Cu) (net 13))
 (segment (start 172 69) (end 184 69) (width 1) (layer F.Cu) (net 14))
 (segment (start 193 66) (end 195.089998 66) (width 1) (layer F.Cu) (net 15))
 (segment (start 195.399999 66.310001) (end 203.558629 66.310001) (width 1) (layer F.Cu) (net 15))
 (segment (start 195.089998 66) (end 195.399999 66.310001) (width 1) (layer F.Cu) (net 15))
 (segment (start 203.558629 66.310001) (end 203.86863 66) (width 1) (layer F.Cu) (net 15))
 (segment (start 203.86863 66) (end 205 66) (width 1) (layer F.Cu) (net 15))
 (segment (start 193 69) (end 205 69) (width 1) (layer F.Cu) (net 16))
 (segment (start 214 66) (end 216.089998 66) (width 1) (layer F.Cu) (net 17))
 (segment (start 216.089998 66) (end 216.399999 66.310001) (width 1) (layer F.Cu) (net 17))
 (segment (start 216.399999 66.310001) (end 224.558629 66.310001) (width 1) (layer F.Cu) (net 17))
 (segment (start 224.558629 66.310001) (end 224.86863 66) (width 1) (layer F.Cu) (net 17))
 (segment (start 224.86863 66) (end 226 66) (width 1) (layer F.Cu) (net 17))
 (segment (start 214 69) (end 226 69) (width 1) (layer F.Cu) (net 18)))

